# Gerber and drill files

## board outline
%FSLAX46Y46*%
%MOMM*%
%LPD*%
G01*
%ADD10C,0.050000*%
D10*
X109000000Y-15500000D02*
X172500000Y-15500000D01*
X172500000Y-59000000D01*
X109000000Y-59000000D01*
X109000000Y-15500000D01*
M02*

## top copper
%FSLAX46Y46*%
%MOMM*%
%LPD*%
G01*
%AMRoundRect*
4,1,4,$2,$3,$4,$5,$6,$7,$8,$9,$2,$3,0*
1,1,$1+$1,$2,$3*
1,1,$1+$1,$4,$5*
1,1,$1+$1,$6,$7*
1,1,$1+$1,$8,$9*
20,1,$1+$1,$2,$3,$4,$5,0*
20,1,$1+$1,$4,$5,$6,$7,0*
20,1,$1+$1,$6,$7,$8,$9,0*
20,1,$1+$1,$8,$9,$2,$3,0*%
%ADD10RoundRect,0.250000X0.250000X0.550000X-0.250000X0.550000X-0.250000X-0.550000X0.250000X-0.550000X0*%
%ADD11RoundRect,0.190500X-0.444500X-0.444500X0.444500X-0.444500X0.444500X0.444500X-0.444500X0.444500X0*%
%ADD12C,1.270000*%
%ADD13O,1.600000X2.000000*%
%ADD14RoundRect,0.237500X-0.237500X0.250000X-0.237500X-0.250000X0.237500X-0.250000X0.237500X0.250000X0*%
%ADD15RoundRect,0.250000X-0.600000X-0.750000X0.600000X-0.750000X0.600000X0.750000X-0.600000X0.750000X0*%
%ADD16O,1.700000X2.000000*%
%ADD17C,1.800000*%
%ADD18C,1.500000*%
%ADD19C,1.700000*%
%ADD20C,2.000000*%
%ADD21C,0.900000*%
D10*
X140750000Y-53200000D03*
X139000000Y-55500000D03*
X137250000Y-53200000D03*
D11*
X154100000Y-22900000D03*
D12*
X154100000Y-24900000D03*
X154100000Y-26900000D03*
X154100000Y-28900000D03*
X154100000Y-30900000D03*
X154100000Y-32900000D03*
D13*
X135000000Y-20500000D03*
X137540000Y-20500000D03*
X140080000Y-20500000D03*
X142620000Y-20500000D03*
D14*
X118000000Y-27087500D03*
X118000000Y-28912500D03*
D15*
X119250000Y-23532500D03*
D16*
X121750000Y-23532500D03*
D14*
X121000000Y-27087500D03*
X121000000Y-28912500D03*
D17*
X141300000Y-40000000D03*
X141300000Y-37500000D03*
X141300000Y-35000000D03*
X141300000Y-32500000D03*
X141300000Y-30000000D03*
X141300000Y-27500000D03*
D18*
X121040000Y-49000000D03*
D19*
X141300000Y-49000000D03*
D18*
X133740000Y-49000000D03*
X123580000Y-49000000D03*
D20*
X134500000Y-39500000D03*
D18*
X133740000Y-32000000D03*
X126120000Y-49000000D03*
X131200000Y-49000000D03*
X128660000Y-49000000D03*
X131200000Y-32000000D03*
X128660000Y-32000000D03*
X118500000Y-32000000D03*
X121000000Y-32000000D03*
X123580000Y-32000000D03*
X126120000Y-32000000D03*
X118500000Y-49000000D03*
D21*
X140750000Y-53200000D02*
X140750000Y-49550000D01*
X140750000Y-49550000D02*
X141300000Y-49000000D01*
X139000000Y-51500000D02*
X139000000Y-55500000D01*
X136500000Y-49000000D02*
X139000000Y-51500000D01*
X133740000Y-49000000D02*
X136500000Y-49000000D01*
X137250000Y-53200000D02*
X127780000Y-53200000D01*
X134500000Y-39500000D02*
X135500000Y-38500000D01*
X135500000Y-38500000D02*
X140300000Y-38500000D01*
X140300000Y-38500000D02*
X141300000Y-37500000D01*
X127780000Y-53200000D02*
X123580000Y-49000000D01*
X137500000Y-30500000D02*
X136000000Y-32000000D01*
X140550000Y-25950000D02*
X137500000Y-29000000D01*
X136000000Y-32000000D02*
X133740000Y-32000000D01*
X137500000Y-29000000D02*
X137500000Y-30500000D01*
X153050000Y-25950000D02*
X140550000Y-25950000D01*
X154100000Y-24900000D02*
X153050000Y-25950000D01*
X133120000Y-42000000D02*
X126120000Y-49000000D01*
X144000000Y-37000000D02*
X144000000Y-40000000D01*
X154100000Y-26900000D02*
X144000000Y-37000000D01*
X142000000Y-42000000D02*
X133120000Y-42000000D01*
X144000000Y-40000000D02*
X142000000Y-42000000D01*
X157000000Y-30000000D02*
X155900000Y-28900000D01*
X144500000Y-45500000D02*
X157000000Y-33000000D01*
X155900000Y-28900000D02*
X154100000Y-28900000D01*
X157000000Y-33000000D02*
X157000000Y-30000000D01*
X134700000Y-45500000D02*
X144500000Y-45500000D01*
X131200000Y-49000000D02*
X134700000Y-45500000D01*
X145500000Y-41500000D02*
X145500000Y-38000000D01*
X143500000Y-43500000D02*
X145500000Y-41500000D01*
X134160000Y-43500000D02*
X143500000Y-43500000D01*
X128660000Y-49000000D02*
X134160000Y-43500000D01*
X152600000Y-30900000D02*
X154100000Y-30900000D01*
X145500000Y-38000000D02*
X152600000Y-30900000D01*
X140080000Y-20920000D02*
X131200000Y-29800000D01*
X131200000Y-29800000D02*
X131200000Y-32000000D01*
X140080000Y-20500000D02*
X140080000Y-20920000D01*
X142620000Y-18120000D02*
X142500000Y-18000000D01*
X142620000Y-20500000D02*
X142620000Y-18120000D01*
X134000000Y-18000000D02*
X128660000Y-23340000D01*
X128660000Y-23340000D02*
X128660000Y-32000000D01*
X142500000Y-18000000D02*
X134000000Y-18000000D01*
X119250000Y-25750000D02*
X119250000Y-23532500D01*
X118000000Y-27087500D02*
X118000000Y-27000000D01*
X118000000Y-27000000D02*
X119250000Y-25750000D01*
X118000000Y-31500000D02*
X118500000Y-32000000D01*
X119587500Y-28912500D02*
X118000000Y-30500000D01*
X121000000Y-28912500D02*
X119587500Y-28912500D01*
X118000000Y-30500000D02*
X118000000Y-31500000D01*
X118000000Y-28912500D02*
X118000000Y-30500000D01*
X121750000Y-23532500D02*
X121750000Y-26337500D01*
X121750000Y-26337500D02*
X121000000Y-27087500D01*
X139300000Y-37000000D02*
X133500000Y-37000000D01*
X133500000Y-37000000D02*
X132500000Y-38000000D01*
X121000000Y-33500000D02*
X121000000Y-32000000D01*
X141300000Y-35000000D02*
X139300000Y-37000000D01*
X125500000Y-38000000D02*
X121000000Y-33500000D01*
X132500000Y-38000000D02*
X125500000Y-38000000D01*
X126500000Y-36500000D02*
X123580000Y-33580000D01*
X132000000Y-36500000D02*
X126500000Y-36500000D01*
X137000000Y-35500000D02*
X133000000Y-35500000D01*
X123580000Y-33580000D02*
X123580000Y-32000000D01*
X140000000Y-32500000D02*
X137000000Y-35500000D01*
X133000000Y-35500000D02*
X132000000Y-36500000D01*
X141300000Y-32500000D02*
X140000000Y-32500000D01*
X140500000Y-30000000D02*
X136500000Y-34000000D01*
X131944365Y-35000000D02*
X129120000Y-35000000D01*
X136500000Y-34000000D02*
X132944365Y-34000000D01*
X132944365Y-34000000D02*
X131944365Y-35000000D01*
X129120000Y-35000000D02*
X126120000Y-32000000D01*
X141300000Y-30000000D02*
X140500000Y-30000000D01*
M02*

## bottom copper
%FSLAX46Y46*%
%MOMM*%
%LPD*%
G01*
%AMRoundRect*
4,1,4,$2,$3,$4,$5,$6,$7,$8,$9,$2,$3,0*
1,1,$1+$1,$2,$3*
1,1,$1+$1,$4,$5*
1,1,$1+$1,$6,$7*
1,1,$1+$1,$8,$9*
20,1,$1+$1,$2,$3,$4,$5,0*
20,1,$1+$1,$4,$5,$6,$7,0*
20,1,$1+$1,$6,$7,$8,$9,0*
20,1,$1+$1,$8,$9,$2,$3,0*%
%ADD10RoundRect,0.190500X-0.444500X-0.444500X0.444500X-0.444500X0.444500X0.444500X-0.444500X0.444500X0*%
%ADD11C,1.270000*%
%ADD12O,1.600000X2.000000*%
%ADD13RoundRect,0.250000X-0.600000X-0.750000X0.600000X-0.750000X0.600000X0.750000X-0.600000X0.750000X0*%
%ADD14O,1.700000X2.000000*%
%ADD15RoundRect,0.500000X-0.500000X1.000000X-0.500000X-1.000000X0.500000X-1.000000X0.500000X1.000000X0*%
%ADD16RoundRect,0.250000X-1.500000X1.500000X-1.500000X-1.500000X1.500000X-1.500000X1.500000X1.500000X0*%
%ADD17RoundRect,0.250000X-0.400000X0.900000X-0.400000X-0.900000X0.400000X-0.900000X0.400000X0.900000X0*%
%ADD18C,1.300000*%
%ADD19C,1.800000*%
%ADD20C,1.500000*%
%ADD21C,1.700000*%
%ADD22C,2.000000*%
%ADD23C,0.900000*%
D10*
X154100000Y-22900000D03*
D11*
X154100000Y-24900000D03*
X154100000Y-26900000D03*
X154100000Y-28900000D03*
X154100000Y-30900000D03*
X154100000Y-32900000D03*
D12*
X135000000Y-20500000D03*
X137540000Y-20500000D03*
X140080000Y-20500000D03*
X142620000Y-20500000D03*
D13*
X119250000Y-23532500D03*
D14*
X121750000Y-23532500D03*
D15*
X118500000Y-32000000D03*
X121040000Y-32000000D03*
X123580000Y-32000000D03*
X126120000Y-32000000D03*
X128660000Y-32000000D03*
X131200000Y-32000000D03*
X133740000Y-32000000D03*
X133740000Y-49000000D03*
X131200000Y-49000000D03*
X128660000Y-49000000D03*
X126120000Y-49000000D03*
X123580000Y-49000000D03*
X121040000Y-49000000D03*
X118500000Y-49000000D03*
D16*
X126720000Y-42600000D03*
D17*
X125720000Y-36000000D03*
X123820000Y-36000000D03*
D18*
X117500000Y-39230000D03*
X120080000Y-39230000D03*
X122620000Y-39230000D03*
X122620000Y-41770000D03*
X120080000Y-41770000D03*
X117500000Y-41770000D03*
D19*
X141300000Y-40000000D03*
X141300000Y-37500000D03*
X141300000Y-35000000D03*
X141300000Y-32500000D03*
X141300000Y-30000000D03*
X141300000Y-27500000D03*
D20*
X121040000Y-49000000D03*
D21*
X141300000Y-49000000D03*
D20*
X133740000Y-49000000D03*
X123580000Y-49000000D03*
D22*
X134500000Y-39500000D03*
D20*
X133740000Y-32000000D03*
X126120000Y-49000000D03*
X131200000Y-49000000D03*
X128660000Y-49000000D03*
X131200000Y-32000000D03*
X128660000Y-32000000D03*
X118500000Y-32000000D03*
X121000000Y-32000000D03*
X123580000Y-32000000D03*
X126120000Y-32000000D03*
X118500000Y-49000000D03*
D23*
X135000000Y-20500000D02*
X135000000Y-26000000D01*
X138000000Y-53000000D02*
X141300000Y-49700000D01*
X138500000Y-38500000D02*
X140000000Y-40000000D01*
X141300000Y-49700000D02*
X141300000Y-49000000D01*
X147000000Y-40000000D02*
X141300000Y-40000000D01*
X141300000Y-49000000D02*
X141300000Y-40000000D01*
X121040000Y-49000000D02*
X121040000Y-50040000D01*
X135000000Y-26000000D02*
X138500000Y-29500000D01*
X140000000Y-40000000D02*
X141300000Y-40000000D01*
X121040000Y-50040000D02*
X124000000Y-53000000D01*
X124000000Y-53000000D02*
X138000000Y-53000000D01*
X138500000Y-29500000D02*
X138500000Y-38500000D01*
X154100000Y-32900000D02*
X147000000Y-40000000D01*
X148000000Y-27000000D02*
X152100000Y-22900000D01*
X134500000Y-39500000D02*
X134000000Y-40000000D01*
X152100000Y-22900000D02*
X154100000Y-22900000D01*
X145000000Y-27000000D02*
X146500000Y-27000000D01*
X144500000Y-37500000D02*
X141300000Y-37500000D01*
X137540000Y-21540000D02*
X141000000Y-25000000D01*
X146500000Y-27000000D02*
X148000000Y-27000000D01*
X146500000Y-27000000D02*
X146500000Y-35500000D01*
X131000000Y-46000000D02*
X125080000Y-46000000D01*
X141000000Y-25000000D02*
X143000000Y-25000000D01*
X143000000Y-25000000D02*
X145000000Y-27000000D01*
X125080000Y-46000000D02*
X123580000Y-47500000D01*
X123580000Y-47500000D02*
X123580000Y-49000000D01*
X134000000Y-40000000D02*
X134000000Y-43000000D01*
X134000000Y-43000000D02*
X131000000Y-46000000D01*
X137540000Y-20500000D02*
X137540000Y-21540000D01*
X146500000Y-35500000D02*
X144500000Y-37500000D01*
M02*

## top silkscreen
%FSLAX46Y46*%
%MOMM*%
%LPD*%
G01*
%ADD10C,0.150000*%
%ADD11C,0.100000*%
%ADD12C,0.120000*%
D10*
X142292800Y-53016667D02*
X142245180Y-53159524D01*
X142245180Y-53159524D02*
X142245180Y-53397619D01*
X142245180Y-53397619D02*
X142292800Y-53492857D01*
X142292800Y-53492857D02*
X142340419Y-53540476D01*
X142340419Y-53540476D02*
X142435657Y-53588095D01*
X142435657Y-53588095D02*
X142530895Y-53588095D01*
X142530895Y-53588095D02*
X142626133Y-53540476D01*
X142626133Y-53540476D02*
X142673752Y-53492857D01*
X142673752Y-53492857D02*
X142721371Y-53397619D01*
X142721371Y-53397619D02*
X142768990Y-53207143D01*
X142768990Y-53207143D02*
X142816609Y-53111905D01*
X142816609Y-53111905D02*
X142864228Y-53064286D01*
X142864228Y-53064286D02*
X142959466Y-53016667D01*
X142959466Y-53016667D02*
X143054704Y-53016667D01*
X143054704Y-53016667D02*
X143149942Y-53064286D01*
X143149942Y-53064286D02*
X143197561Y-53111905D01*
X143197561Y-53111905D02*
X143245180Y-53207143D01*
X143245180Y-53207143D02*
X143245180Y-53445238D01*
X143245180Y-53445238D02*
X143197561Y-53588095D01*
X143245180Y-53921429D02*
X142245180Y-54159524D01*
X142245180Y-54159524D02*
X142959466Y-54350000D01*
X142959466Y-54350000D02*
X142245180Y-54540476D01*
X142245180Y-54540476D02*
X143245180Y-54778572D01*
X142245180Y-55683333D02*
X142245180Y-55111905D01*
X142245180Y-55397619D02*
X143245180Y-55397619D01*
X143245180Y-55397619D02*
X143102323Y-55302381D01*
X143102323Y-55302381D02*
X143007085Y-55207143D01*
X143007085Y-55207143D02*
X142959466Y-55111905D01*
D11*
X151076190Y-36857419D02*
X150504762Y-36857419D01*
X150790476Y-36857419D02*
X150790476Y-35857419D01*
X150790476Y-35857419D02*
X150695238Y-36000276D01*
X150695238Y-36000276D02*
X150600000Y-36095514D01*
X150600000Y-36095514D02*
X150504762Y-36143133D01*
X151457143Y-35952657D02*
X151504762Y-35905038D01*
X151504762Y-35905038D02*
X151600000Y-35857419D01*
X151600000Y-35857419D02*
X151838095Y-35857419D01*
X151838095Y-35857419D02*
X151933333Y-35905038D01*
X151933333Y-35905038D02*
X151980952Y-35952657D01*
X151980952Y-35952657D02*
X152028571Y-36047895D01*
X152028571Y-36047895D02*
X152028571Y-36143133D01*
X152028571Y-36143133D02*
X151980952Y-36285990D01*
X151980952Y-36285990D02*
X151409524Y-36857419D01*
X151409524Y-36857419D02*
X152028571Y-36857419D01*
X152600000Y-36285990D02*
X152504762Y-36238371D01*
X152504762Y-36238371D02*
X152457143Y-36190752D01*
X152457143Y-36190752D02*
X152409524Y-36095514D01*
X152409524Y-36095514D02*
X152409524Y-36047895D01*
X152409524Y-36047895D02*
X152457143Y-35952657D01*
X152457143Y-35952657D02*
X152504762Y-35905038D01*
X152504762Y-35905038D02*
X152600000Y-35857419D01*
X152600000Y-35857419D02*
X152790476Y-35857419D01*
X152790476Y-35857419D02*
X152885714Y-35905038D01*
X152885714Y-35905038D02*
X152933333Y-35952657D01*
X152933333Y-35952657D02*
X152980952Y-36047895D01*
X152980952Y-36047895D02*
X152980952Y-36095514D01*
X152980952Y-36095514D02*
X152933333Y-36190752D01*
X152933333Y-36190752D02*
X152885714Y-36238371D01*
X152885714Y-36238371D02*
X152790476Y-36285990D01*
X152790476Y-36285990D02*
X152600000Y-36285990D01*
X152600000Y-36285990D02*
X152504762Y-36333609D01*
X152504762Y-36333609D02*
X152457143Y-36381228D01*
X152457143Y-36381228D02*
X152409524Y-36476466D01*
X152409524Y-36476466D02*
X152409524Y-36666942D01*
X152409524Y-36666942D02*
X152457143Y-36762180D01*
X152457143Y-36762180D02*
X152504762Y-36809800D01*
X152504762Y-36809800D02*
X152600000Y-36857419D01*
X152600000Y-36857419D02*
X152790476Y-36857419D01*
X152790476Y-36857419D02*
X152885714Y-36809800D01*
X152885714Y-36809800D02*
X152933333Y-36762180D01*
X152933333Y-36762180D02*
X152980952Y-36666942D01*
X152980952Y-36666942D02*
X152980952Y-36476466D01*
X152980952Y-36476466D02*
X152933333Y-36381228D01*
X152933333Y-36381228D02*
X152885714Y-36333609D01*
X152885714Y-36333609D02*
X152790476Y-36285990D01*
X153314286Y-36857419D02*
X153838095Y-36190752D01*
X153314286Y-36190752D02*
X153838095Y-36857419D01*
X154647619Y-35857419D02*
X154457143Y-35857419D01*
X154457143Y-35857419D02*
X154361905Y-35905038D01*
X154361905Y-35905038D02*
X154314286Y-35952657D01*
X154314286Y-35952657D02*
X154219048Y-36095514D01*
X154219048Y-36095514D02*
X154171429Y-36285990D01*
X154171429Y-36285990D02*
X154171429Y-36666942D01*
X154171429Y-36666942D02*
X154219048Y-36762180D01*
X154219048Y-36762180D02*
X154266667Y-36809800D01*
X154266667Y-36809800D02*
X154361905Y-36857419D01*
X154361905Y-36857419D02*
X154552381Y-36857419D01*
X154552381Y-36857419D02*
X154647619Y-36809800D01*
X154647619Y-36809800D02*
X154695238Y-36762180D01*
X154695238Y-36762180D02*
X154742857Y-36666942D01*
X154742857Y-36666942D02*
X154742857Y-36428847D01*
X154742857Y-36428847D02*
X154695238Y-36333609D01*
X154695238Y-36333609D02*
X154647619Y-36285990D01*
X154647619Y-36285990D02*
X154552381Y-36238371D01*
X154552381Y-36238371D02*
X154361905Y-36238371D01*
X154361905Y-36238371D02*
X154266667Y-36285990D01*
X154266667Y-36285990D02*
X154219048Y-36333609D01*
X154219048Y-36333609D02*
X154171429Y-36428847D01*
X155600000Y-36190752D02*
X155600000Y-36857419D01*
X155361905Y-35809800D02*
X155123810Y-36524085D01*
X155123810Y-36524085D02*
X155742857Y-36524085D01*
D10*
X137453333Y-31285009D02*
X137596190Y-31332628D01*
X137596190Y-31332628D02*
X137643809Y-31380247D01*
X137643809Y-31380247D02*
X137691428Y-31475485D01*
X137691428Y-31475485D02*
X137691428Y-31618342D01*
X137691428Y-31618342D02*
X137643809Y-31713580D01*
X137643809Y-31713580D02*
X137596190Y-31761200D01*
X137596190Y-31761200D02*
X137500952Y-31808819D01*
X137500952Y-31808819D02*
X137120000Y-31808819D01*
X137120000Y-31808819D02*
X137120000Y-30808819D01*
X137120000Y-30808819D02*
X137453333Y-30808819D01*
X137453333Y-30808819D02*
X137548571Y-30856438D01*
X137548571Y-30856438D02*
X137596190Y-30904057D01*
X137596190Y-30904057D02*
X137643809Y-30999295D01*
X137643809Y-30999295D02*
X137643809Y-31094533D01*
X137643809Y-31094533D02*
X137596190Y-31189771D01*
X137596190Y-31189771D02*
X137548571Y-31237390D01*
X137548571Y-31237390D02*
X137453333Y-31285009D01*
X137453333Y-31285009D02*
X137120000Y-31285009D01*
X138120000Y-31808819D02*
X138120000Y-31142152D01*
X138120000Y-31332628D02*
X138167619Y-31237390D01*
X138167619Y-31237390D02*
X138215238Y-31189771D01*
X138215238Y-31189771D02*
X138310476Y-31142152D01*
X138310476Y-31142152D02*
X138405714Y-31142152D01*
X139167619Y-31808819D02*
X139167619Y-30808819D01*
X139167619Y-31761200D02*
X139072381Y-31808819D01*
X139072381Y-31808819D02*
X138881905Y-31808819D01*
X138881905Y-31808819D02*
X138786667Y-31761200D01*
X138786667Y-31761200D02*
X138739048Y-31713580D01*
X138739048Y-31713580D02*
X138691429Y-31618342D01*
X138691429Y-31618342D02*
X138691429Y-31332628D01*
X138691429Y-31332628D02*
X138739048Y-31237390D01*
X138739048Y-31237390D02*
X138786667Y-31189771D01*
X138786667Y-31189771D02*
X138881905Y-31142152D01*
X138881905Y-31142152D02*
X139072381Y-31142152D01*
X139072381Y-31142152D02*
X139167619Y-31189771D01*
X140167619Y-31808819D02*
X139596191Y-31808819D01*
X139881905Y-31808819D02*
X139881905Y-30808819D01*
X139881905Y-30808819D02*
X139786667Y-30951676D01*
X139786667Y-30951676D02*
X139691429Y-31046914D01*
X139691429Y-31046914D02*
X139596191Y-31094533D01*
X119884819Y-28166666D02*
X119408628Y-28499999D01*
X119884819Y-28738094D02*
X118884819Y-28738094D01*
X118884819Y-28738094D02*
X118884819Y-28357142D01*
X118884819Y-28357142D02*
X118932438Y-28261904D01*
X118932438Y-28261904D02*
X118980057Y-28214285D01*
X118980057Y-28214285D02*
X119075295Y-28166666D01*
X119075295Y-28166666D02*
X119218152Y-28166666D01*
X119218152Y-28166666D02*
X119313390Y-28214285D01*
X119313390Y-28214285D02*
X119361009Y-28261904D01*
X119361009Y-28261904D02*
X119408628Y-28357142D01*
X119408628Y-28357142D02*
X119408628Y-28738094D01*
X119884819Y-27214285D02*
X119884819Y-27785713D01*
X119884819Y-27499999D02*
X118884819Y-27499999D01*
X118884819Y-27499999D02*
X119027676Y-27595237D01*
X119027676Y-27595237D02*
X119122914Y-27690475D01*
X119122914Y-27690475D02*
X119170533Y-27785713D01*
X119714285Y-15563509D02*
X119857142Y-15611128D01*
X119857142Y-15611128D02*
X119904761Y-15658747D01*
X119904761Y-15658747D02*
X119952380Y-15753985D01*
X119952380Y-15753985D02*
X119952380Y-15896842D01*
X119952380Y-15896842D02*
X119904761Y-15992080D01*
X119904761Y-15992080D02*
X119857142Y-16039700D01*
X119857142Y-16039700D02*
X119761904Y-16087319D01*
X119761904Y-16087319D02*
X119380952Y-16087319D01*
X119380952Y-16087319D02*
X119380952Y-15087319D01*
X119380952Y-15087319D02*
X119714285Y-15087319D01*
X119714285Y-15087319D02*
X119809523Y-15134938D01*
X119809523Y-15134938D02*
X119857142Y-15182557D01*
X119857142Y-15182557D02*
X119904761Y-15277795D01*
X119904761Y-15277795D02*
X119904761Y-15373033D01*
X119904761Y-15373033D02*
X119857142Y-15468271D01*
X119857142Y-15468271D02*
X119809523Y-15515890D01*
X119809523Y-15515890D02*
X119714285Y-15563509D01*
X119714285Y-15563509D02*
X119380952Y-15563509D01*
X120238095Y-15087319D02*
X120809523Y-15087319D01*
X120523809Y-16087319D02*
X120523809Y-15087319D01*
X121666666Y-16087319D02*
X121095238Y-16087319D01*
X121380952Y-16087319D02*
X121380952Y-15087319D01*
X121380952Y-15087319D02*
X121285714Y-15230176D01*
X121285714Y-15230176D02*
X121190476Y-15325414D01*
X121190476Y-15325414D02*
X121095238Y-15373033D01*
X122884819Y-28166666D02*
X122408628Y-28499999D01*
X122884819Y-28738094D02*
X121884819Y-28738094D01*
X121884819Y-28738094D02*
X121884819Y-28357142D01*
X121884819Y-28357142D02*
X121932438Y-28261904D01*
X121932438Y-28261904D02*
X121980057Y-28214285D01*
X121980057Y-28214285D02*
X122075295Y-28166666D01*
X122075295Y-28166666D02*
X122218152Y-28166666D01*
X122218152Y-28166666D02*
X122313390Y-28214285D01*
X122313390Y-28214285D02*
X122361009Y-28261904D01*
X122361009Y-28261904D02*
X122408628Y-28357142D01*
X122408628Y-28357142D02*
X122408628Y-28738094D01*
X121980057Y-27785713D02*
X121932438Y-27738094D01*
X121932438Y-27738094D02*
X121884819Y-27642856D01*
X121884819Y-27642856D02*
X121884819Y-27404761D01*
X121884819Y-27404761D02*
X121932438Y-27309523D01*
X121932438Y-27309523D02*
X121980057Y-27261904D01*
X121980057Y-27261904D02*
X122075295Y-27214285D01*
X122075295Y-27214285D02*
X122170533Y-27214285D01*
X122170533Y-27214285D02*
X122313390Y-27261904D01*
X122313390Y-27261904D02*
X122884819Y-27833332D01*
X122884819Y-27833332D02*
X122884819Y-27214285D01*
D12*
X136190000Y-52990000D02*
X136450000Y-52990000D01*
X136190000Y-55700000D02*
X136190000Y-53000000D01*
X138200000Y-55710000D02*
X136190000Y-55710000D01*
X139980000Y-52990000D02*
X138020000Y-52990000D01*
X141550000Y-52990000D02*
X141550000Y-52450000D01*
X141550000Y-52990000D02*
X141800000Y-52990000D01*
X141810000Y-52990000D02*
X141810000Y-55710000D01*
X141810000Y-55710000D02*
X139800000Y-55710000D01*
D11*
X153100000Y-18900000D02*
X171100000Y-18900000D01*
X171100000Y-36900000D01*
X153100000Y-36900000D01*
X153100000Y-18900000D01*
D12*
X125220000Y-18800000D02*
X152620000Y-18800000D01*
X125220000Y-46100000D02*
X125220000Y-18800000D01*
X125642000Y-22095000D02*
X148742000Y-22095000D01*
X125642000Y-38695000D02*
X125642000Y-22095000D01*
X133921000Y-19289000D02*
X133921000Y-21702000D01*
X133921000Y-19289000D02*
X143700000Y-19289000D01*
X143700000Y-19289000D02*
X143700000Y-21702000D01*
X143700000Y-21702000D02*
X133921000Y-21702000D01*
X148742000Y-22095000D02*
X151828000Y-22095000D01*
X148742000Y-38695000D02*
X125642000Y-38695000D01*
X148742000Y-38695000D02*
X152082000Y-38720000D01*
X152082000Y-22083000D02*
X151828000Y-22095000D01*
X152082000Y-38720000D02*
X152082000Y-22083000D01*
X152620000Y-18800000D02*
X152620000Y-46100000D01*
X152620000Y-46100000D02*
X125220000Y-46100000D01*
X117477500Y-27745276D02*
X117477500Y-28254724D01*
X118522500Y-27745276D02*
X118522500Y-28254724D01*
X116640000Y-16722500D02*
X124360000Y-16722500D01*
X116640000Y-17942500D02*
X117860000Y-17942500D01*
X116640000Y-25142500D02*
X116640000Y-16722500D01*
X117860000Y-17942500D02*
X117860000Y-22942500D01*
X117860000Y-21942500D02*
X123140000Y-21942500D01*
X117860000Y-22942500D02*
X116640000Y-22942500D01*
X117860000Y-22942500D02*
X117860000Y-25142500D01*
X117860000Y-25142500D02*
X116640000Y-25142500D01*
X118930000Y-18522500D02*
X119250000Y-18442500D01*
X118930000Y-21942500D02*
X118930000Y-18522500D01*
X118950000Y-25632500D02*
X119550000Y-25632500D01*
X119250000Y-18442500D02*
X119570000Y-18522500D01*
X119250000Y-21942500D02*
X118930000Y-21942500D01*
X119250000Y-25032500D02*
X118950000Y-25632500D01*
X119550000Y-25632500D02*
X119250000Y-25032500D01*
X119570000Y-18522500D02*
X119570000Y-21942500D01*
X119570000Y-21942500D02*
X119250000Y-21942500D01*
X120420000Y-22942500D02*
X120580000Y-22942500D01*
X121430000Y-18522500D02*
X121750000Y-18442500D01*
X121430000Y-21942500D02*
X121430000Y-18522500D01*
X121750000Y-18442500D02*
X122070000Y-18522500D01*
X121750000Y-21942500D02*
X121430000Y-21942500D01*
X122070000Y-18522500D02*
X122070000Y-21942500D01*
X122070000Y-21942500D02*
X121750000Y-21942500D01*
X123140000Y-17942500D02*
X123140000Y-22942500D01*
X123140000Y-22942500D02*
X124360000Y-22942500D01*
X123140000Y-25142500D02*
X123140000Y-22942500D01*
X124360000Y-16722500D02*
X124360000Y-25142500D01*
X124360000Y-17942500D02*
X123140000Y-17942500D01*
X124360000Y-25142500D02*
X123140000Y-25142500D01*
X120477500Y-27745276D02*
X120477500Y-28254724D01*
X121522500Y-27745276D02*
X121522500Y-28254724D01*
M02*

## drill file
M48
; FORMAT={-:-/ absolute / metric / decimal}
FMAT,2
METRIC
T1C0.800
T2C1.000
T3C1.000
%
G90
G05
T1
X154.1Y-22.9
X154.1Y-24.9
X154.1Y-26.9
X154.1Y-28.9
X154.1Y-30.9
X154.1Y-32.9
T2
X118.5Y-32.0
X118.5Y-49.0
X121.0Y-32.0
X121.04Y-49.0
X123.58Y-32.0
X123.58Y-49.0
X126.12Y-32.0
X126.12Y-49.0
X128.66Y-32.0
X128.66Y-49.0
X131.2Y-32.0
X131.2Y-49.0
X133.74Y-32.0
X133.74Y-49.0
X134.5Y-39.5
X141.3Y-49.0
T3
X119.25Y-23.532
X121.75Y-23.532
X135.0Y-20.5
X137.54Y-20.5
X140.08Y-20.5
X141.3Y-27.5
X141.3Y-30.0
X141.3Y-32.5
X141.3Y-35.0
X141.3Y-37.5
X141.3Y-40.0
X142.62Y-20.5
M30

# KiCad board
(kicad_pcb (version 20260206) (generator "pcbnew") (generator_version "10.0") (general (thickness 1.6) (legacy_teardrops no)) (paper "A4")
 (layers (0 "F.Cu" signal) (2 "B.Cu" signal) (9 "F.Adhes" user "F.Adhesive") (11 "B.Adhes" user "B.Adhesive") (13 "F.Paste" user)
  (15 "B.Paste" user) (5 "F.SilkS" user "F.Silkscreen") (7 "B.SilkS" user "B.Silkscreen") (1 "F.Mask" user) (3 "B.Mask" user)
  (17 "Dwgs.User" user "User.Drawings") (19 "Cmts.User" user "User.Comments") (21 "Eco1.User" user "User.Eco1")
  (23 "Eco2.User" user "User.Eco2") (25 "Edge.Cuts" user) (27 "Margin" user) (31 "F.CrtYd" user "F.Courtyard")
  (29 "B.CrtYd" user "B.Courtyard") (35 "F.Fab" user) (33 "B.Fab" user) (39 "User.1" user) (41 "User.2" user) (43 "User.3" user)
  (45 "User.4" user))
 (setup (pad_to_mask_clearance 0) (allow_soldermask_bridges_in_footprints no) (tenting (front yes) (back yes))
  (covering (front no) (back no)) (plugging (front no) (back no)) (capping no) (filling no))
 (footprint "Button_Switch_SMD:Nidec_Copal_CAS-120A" (layer "F.Cu") (at 139 54.35 -90)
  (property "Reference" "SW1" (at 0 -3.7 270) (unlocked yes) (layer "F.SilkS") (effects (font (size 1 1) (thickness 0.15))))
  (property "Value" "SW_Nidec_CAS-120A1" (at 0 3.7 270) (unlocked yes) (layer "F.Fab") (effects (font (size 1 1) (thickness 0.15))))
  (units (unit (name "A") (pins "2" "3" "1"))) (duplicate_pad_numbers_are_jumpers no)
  (fp_line (start -1.36 2.81) (end -1.36 2.55) (stroke (width 0.12) (type solid)) (layer "F.SilkS"))
  (fp_line (start 1.35 2.81) (end -1.35 2.81) (stroke (width 0.12) (type solid)) (layer "F.SilkS"))
  (fp_line (start 1.36 0.8) (end 1.36 2.81) (stroke (width 0.12) (type solid)) (layer "F.SilkS"))
  (fp_line (start -1.36 -0.98) (end -1.36 0.98) (stroke (width 0.12) (type solid)) (layer "F.SilkS"))
  (fp_line (start -1.36 -2.55) (end -1.9 -2.55) (stroke (width 0.12) (type default)) (layer "F.SilkS"))
  (fp_line (start -1.36 -2.55) (end -1.36 -2.8) (stroke (width 0.12) (type solid)) (layer "F.SilkS"))
  (fp_line (start -1.36 -2.81) (end 1.36 -2.81) (stroke (width 0.12) (type solid)) (layer "F.SilkS"))
  (fp_line (start 1.36 -2.81) (end 1.36 -0.8) (stroke (width 0.12) (type solid)) (layer "F.SilkS"))
  (pad "1" smd roundrect (at -1.15 -1.75 180) (size 1 1.6) (layers "F.Cu" "F.Mask" "F.Paste") (roundrect_rratio 0.25) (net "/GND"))
  (pad "2" smd roundrect (at 1.15 0 180) (size 1 1.6) (layers "F.Cu" "F.Mask" "F.Paste") (roundrect_rratio 0.25) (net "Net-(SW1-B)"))
  (pad "3" smd roundrect (at -1.15 1.75 180) (size 1 1.6) (layers "F.Cu" "F.Mask" "F.Paste") (roundrect_rratio 0.25) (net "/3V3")))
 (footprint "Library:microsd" (layer "F.Cu") (at 153.1 36.9)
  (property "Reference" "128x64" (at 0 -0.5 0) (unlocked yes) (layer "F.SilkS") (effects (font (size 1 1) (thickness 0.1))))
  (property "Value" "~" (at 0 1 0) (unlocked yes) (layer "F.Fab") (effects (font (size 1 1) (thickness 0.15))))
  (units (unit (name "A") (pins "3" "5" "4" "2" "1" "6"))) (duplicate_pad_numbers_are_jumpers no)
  (fp_rect (start 0 -18) (end 18 0) (stroke (width 0.1) (type default)) (fill no) (layer "F.SilkS"))
  (pad "1" thru_hole roundrect (at 1 -14) (size 1.27 1.27) (drill 0.8) (layers "*.Cu" "*.Mask") (remove_unused_layers no)
   (roundrect_rratio 0.15) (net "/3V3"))
  (pad "2" thru_hole circle (at 1 -12) (size 1.27 1.27) (drill 0.8) (layers "*.Cu" "*.Mask") (remove_unused_layers no) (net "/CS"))
  (pad "3" thru_hole circle (at 1 -10) (size 1.27 1.27) (drill 0.8) (layers "*.Cu" "*.Mask") (remove_unused_layers no) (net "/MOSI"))
  (pad "4" thru_hole circle (at 1 -8) (size 1.27 1.27) (drill 0.8) (layers "*.Cu" "*.Mask") (remove_unused_layers no) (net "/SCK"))
  (pad "5" thru_hole circle (at 1 -6) (size 1.27 1.27) (drill 0.8) (layers "*.Cu" "*.Mask") (remove_unused_layers no) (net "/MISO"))
  (pad "6" thru_hole circle (at 1 -4) (size 1.27 1.27) (drill 0.8) (layers "*.Cu" "*.Mask") (remove_unused_layers no) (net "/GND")))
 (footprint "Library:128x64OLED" (layer "F.Cu") (at 138.62 31.1)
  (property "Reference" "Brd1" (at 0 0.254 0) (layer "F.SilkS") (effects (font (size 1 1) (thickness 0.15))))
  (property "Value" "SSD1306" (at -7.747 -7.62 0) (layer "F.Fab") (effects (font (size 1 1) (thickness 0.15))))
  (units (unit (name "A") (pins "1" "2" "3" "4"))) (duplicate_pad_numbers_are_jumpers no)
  (fp_line (start -13.4 -12.3) (end 14 -12.3) (stroke (width 0.12) (type solid)) (layer "F.SilkS"))
  (fp_line (start -13.4 15) (end -13.4 -12.3) (stroke (width 0.12) (type solid)) (layer "F.SilkS"))
  (fp_line (start -12.978 -9.005) (end 10.122 -9.005) (stroke (width 0.12) (type solid)) (layer "F.SilkS"))
  (fp_line (start -12.978 7.595) (end -12.978 -9.005) (stroke (width 0.12) (type solid)) (layer "F.SilkS"))
  (fp_line (start -4.699 -11.811) (end -4.699 -9.398) (stroke (width 0.12) (type solid)) (layer "F.SilkS"))
  (fp_line (start -4.699 -11.811) (end 5.08 -11.811) (stroke (width 0.12) (type solid)) (layer "F.SilkS"))
  (fp_line (start 5.08 -11.811) (end 5.08 -9.398) (stroke (width 0.12) (type solid)) (layer "F.SilkS"))
  (fp_line (start 5.08 -9.398) (end -4.699 -9.398) (stroke (width 0.12) (type solid)) (layer "F.SilkS"))
  (fp_line (start 10.122 -9.005) (end 13.208 -9.005) (stroke (width 0.12) (type solid)) (layer "F.SilkS"))
  (fp_line (start 10.122 7.595) (end -12.978 7.595) (stroke (width 0.12) (type solid)) (layer "F.SilkS"))
  (fp_line (start 10.122 7.595) (end 13.462 7.62) (stroke (width 0.12) (type solid)) (layer "F.SilkS"))
  (fp_line (start 13.462 -9.017) (end 13.208 -9.005) (stroke (width 0.12) (type solid)) (layer "F.SilkS"))
  (fp_line (start 13.462 7.62) (end 13.462 -9.017) (stroke (width 0.12) (type solid)) (layer "F.SilkS"))
  (fp_line (start 14 -12.3) (end 14 15) (stroke (width 0.12) (type solid)) (layer "F.SilkS"))
  (fp_line (start 14 15) (end -13.4 15) (stroke (width 0.12) (type solid)) (layer "F.SilkS"))
  (pad "1" thru_hole oval (at -3.62 -10.6 90) (size 2 1.6) (drill 1) (layers "*.Cu" "*.Mask") (remove_unused_layers no) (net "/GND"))
  (pad "2" thru_hole oval (at -1.08 -10.6 90) (size 2 1.6) (drill 1) (layers "*.Cu" "*.Mask") (remove_unused_layers no) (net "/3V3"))
  (pad "3" thru_hole oval (at 1.46 -10.6 90) (size 2 1.6) (drill 1) (layers "*.Cu" "*.Mask") (remove_unused_layers no) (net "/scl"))
  (pad "4" thru_hole oval (at 4 -10.6 90) (size 2 1.6) (drill 1) (layers "*.Cu" "*.Mask") (remove_unused_layers no) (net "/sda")))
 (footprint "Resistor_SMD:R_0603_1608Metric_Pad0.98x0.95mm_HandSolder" (layer "F.Cu") (at 118 28 -90)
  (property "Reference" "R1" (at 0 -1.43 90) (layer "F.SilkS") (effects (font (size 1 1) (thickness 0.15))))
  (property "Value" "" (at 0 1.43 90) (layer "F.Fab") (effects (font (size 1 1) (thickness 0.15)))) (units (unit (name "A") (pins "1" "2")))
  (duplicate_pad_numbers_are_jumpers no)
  (fp_line (start -0.254724 0.5225) (end 0.254724 0.5225) (stroke (width 0.12) (type solid)) (layer "F.SilkS"))
  (fp_line (start -0.254724 -0.5225) (end 0.254724 -0.5225) (stroke (width 0.12) (type solid)) (layer "F.SilkS"))
  (pad "1" smd roundrect (at -0.9125 0 270) (size 0.975 0.95) (layers "F.Cu" "F.Mask" "F.Paste") (roundrect_rratio 0.25) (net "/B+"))
  (pad "2" smd roundrect (at 0.9125 0 270) (size 0.975 0.95) (layers "F.Cu" "F.Mask" "F.Paste") (roundrect_rratio 0.25) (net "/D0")))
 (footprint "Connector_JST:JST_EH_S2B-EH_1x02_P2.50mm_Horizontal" (layer "F.Cu") (at 119.25 23.5325)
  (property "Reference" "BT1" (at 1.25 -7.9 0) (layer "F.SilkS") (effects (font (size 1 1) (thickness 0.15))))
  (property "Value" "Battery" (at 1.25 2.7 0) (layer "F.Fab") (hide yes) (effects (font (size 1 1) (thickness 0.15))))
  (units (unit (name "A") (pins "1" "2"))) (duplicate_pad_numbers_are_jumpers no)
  (fp_line (start -2.61 -6.81) (end 5.11 -6.81) (stroke (width 0.12) (type solid)) (layer "F.SilkS"))
  (fp_line (start -2.61 -5.59) (end -1.39 -5.59) (stroke (width 0.12) (type solid)) (layer "F.SilkS"))
  (fp_line (start -2.61 1.61) (end -2.61 -6.81) (stroke (width 0.12) (type solid)) (layer "F.SilkS"))
  (fp_line (start -1.39 -5.59) (end -1.39 -0.59) (stroke (width 0.12) (type solid)) (layer "F.SilkS"))
  (fp_line (start -1.39 -1.59) (end 3.89 -1.59) (stroke (width 0.12) (type solid)) (layer "F.SilkS"))
  (fp_line (start -1.39 -0.59) (end -2.61 -0.59) (stroke (width 0.12) (type solid)) (layer "F.SilkS"))
  (fp_line (start -1.39 -0.59) (end -1.39 1.61) (stroke (width 0.12) (type solid)) (layer "F.SilkS"))
  (fp_line (start -1.39 1.61) (end -2.61 1.61) (stroke (width 0.12) (type solid)) (layer "F.SilkS"))
  (fp_line (start -0.32 -5.01) (end 0 -5.09) (stroke (width 0.12) (type solid)) (layer "F.SilkS"))
  (fp_line (start -0.32 -1.59) (end -0.32 -5.01) (stroke (width 0.12) (type solid)) (layer "F.SilkS"))
  (fp_line (start -0.3 2.1) (end 0.3 2.1) (stroke (width 0.12) (type solid)) (layer "F.SilkS"))
  (fp_line (start 0 -5.09) (end 0.32 -5.01) (stroke (width 0.12) (type solid)) (layer "F.SilkS"))
  (fp_line (start 0 -1.59) (end -0.32 -1.59) (stroke (width 0.12) (type solid)) (layer "F.SilkS"))
  (fp_line (start 0 1.5) (end -0.3 2.1) (stroke (width 0.12) (type solid)) (layer "F.SilkS"))
  (fp_line (start 0.3 2.1) (end 0 1.5) (stroke (width 0.12) (type solid)) (layer "F.SilkS"))
  (fp_line (start 0.32 -5.01) (end 0.32 -1.59) (stroke (width 0.12) (type solid)) (layer "F.SilkS"))
  (fp_line (start 0.32 -1.59) (end 0 -1.59) (stroke (width 0.12) (type solid)) (layer "F.SilkS"))
  (fp_line (start 1.17 -0.59) (end 1.33 -0.59) (stroke (width 0.12) (type solid)) (layer "F.SilkS"))
  (fp_line (start 2.18 -5.01) (end 2.5 -5.09) (stroke (width 0.12) (type solid)) (layer "F.SilkS"))
  (fp_line (start 2.18 -1.59) (end 2.18 -5.01) (stroke (width 0.12) (type solid)) (layer "F.SilkS"))
  (fp_line (start 2.5 -5.09) (end 2.82 -5.01) (stroke (width 0.12) (type solid)) (layer "F.SilkS"))
  (fp_line (start 2.5 -1.59) (end 2.18 -1.59) (stroke (width 0.12) (type solid)) (layer "F.SilkS"))
  (fp_line (start 2.82 -5.01) (end 2.82 -1.59) (stroke (width 0.12) (type solid)) (layer "F.SilkS"))
  (fp_line (start 2.82 -1.59) (end 2.5 -1.59) (stroke (width 0.12) (type solid)) (layer "F.SilkS"))
  (fp_line (start 3.89 -5.59) (end 3.89 -0.59) (stroke (width 0.12) (type solid)) (layer "F.SilkS"))
  (fp_line (start 3.89 -0.59) (end 5.11 -0.59) (stroke (width 0.12) (type solid)) (layer "F.SilkS"))
  (fp_line (start 3.89 1.61) (end 3.89 -0.59) (stroke (width 0.12) (type solid)) (layer "F.SilkS"))
  (fp_line (start 5.11 -6.81) (end 5.11 1.61) (stroke (width 0.12) (type solid)) (layer "F.SilkS"))
  (fp_line (start 5.11 -5.59) (end 3.89 -5.59) (stroke (width 0.12) (type solid)) (layer "F.SilkS"))
  (fp_line (start 5.11 1.61) (end 3.89 1.61) (stroke (width 0.12) (type solid)) (layer "F.SilkS"))
  (pad "1" thru_hole roundrect (at 0 0) (size 1.7 2) (drill 1) (layers "*.Cu" "*.Mask") (remove_unused_layers no)
   (roundrect_rratio 0.147059) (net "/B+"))
  (pad "2" thru_hole oval (at 2.5 0) (size 1.7 2) (drill 1) (layers "*.Cu" "*.Mask") (remove_unused_layers no) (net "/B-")))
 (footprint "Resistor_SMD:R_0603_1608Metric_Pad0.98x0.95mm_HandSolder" (layer "F.Cu") (at 121 28 -90)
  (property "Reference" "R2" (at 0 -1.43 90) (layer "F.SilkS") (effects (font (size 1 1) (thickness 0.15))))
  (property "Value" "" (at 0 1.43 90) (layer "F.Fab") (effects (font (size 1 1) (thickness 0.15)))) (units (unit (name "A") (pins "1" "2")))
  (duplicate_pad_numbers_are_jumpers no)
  (fp_line (start -0.254724 0.5225) (end 0.254724 0.5225) (stroke (width 0.12) (type solid)) (layer "F.SilkS"))
  (fp_line (start -0.254724 -0.5225) (end 0.254724 -0.5225) (stroke (width 0.12) (type solid)) (layer "F.SilkS"))
  (pad "1" smd roundrect (at -0.9125 0 270) (size 0.975 0.95) (layers "F.Cu" "F.Mask" "F.Paste") (roundrect_rratio 0.25) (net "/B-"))
  (pad "2" smd roundrect (at 0.9125 0 270) (size 0.975 0.95) (layers "F.Cu" "F.Mask" "F.Paste") (roundrect_rratio 0.25) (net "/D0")))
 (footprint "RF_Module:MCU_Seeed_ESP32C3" (layer "B.Cu") (at 126.12 40.5 -90)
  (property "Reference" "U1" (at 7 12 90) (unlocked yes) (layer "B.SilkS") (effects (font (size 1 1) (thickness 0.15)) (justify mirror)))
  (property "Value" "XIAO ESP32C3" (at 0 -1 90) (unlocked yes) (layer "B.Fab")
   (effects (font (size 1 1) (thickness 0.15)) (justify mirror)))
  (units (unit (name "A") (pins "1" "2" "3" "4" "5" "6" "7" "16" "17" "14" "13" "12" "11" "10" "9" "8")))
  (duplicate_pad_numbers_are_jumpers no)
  (pad "" smd roundrect (at 1.1 -1.6 270) (size 1.5 1.5) (layers "B.Paste") (roundrect_rratio 0.1666666667))
  (pad "" smd roundrect (at 1.1 0.4 270) (size 1.5 1.5) (layers "B.Paste") (roundrect_rratio 0.1666666667))
  (pad "" smd roundrect (at 3.1 -1.6 270) (size 1.5 1.5) (layers "B.Paste") (roundrect_rratio 0.1666666667))
  (pad "" smd roundrect (at 3.1 0.4 270) (size 1.5 1.5) (layers "B.Paste") (roundrect_rratio 0.1666666667))
  (pad "1" smd roundrect (at -8.5 7.62 270) (size 3 2) (layers "B.Cu" "B.Mask" "B.Paste") (roundrect_rratio 0.25) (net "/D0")
   (thermal_bridge_angle 45))
  (pad "2" smd roundrect (at -8.5 5.08 270) (size 3 2) (layers "B.Cu" "B.Mask" "B.Paste") (roundrect_rratio 0.25) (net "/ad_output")
   (thermal_bridge_angle 45))
  (pad "3" smd roundrect (at -8.5 2.54 270) (size 3 2) (layers "B.Cu" "B.Mask" "B.Paste") (roundrect_rratio 0.25) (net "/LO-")
   (thermal_bridge_angle 45))
  (pad "4" smd roundrect (at -8.5 0 270) (size 3 2) (layers "B.Cu" "B.Mask" "B.Paste") (roundrect_rratio 0.25) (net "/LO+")
   (thermal_bridge_angle 45))
  (pad "5" smd roundrect (at -8.5 -2.54 270) (size 3 2) (layers "B.Cu" "B.Mask" "B.Paste") (roundrect_rratio 0.25) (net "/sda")
   (thermal_bridge_angle 45))
  (pad "6" smd roundrect (at -8.5 -5.08 270) (size 3 2) (layers "B.Cu" "B.Mask" "B.Paste") (roundrect_rratio 0.25) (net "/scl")
   (thermal_bridge_angle 45))
  (pad "7" smd roundrect (at -8.5 -7.62 270) (size 3 2) (layers "B.Cu" "B.Mask" "B.Paste") (roundrect_rratio 0.25) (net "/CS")
   (thermal_bridge_angle 45))
  (pad "8" smd roundrect (at 8.5 -7.62 270) (size 3 2) (layers "B.Cu" "B.Mask" "B.Paste") (roundrect_rratio 0.25) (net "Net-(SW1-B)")
   (thermal_bridge_angle 45))
  (pad "9" smd roundrect (at 8.5 -5.08 270) (size 3 2) (layers "B.Cu" "B.Mask" "B.Paste") (roundrect_rratio 0.25) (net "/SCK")
   (thermal_bridge_angle 45))
  (pad "10" smd roundrect (at 8.5 -2.54 270) (size 3 2) (layers "B.Cu" "B.Mask" "B.Paste") (roundrect_rratio 0.25) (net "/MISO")
   (thermal_bridge_angle 45))
  (pad "11" smd roundrect (at 8.5 0 270) (size 3 2) (layers "B.Cu" "B.Mask" "B.Paste") (roundrect_rratio 0.25) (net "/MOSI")
   (thermal_bridge_angle 45))
  (pad "12" smd roundrect (at 8.5 2.54 270) (size 3 2) (layers "B.Cu" "B.Mask" "B.Paste") (roundrect_rratio 0.25) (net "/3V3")
   (thermal_bridge_angle 45))
  (pad "13" smd roundrect (at 8.5 5.08 270) (size 3 2) (layers "B.Cu" "B.Mask" "B.Paste") (roundrect_rratio 0.25) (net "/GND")
   (thermal_bridge_angle 45))
  (pad "14" smd roundrect (at 8.5 7.62 270) (size 3 2) (layers "B.Cu" "B.Mask" "B.Paste") (roundrect_rratio 0.25)
   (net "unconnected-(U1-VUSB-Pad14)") (thermal_bridge_angle 45))
  (pad "15" smd roundrect (at 2.1 -0.6 270) (size 3.5 3.5) (layers "B.Cu" "B.Mask") (roundrect_rratio 0.07142857143))
  (pad "16" smd roundrect (at -4.5 0.4 270) (size 2.3 1.3) (layers "B.Cu" "B.Mask" "B.Paste") (roundrect_rratio 0.1923076923) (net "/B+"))
  (pad "17" smd roundrect (at -4.5 2.3 270) (size 2.3 1.3) (layers "B.Cu" "B.Mask" "B.Paste") (roundrect_rratio 0.1923076923) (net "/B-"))
  (pad "18" smd circle (at -1.27 8.62 270) (size 1.3 1.3) (layers "B.Cu" "B.Mask" "B.Paste"))
  (pad "19" smd circle (at -1.27 6.04 270) (size 1.3 1.3) (layers "B.Cu" "B.Mask" "B.Paste"))
  (pad "20" smd circle (at -1.27 3.5 270) (size 1.3 1.3) (layers "B.Cu" "B.Mask" "B.Paste"))
  (pad "21" smd circle (at 1.27 3.5 270) (size 1.3 1.3) (layers "B.Cu" "B.Mask" "B.Paste"))
  (pad "22" smd circle (at 1.27 6.04 270) (size 1.3 1.3) (layers "B.Cu" "B.Mask" "B.Paste"))
  (pad "23" smd circle (at 1.27 8.62 270) (size 1.3 1.3) (layers "B.Cu" "B.Mask" "B.Paste")))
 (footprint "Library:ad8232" (layer "B.Cu") (at 140.1 19)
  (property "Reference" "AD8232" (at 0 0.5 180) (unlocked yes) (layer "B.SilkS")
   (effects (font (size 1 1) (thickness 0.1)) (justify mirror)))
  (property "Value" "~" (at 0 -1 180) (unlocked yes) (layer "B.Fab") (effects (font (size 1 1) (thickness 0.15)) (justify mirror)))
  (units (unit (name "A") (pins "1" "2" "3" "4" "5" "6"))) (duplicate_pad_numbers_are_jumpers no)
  (pad "1" thru_hole circle (at 1.2 21) (size 1.8 1.8) (drill 1) (layers "*.Cu" "*.Mask") (remove_unused_layers no) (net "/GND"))
  (pad "2" thru_hole circle (at 1.2 18.5) (size 1.8 1.8) (drill 1) (layers "*.Cu" "*.Mask") (remove_unused_layers no) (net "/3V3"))
  (pad "3" thru_hole circle (at 1.2 16) (size 1.8 1.8) (drill 1) (layers "*.Cu" "*.Mask") (remove_unused_layers no) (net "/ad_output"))
  (pad "4" thru_hole circle (at 1.2 13.5) (size 1.8 1.8) (drill 1) (layers "*.Cu" "*.Mask") (remove_unused_layers no) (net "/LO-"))
  (pad "5" thru_hole circle (at 1.2 11) (size 1.8 1.8) (drill 1) (layers "*.Cu" "*.Mask") (remove_unused_layers no) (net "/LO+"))
  (pad "6" thru_hole circle (at 1.2 8.5) (size 1.8 1.8) (drill 1) (layers "*.Cu" "*.Mask") (remove_unused_layers no)
   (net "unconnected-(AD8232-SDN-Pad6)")))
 (gr_rect (start 109 15.5) (end 172.5 59) (stroke (width 0.05) (type default)) (fill no) (layer "Edge.Cuts"))
 (segment (start 140.75 53.2) (end 140.75 49.55) (width 0.9) (layer "F.Cu") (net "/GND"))
 (segment (start 140.75 49.55) (end 141.3 49) (width 0.9) (layer "F.Cu") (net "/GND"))
 (via (at 121.04 49) (size 1.5) (drill 1) (layers "F.Cu" "B.Cu") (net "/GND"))
 (via (at 141.3 49) (size 1.7) (drill 1) (layers "F.Cu" "B.Cu") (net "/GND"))
 (segment (start 135 20.5) (end 135 26) (width 0.9) (layer "B.Cu") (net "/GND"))
 (segment (start 138 53) (end 141.3 49.7) (width 0.9) (layer "B.Cu") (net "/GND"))
 (segment (start 138.5 38.5) (end 140 40) (width 0.9) (layer "B.Cu") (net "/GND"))
 (segment (start 141.3 49.7) (end 141.3 49) (width 0.9) (layer "B.Cu") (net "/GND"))
 (segment (start 147 40) (end 141.3 40) (width 0.9) (layer "B.Cu") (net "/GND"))
 (segment (start 141.3 49) (end 141.3 40) (width 0.9) (layer "B.Cu") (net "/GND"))
 (segment (start 121.04 49) (end 121.04 50.04) (width 0.9) (layer "B.Cu") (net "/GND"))
 (segment (start 135 26) (end 138.5 29.5) (width 0.9) (layer "B.Cu") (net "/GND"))
 (segment (start 140 40) (end 141.3 40) (width 0.9) (layer "B.Cu") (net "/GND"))
 (segment (start 121.04 50.04) (end 124 53) (width 0.9) (layer "B.Cu") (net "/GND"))
 (segment (start 124 53) (end 138 53) (width 0.9) (layer "B.Cu") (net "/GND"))
 (segment (start 138.5 29.5) (end 138.5 38.5) (width 0.9) (layer "B.Cu") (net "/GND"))
 (segment (start 154.1 32.9) (end 147 40) (width 0.9) (layer "B.Cu") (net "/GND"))
 (segment (start 139 51.5) (end 139 55.5) (width 0.9) (layer "F.Cu") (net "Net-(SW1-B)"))
 (segment (start 136.5 49) (end 139 51.5) (width 0.9) (layer "F.Cu") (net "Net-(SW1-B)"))
 (segment (start 133.74 49) (end 136.5 49) (width 0.9) (layer "F.Cu") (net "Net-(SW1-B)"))
 (via (at 133.74 49) (size 1.5) (drill 1) (layers "F.Cu" "B.Cu") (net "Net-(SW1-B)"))
 (segment (start 137.25 53.2) (end 127.78 53.2) (width 0.9) (layer "F.Cu") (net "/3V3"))
 (segment (start 134.5 39.5) (end 135.5 38.5) (width 0.9) (layer "F.Cu") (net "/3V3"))
 (segment (start 135.5 38.5) (end 140.3 38.5) (width 0.9) (layer "F.Cu") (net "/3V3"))
 (segment (start 140.3 38.5) (end 141.3 37.5) (width 0.9) (layer "F.Cu") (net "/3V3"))
 (segment (start 127.78 53.2) (end 123.58 49) (width 0.9) (layer "F.Cu") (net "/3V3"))
 (via (at 123.58 49) (size 1.5) (drill 1) (layers "F.Cu" "B.Cu") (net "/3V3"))
 (via (at 134.5 39.5) (size 2) (drill 1) (layers "F.Cu" "B.Cu") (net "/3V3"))
 (segment (start 148 27) (end 152.1 22.9) (width 0.9) (layer "B.Cu") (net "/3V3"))
 (segment (start 134.5 39.5) (end 134 40) (width 0.9) (layer "B.Cu") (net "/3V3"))
 (segment (start 152.1 22.9) (end 154.1 22.9) (width 0.9) (layer "B.Cu") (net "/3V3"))
 (segment (start 145 27) (end 146.5 27) (width 0.9) (layer "B.Cu") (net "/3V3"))
 (segment (start 144.5 37.5) (end 141.3 37.5) (width 0.9) (layer "B.Cu") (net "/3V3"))
 (segment (start 137.54 21.54) (end 141 25) (width 0.9) (layer "B.Cu") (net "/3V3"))
 (segment (start 146.5 27) (end 148 27) (width 0.9) (layer "B.Cu") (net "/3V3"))
 (segment (start 146.5 27) (end 146.5 35.5) (width 0.9) (layer "B.Cu") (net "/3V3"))
 (segment (start 131 46) (end 125.08 46) (width 0.9) (layer "B.Cu") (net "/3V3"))
 (segment (start 141 25) (end 143 25) (width 0.9) (layer "B.Cu") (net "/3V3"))
 (segment (start 143 25) (end 145 27) (width 0.9) (layer "B.Cu") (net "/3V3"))
 (segment (start 125.08 46) (end 123.58 47.5) (width 0.9) (layer "B.Cu") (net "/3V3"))
 (segment (start 123.58 47.5) (end 123.58 49) (width 0.9) (layer "B.Cu") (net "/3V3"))
 (segment (start 134 40) (end 134 43) (width 0.9) (layer "B.Cu") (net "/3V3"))
 (segment (start 134 43) (end 131 46) (width 0.9) (layer "B.Cu") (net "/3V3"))
 (segment (start 137.54 20.5) (end 137.54 21.54) (width 0.9) (layer "B.Cu") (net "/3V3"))
 (segment (start 146.5 35.5) (end 144.5 37.5) (width 0.9) (layer "B.Cu") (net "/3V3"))
 (segment (start 137.5 30.5) (end 136 32) (width 0.9) (layer "F.Cu") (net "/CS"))
 (segment (start 140.55 25.95) (end 137.5 29) (width 0.9) (layer "F.Cu") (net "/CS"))
 (segment (start 136 32) (end 133.74 32) (width 0.9) (layer "F.Cu") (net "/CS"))
 (segment (start 137.5 29) (end 137.5 30.5) (width 0.9) (layer "F.Cu") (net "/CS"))
 (segment (start 153.05 25.95) (end 140.55 25.95) (width 0.9) (layer "F.Cu") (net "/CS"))
 (segment (start 154.1 24.9) (end 153.05 25.95) (width 0.9) (layer "F.Cu") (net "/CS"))
 (via (at 133.74 32) (size 1.5) (drill 1) (layers "F.Cu" "B.Cu") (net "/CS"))
 (segment (start 133.12 42) (end 126.12 49) (width 0.9) (layer "F.Cu") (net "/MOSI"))
 (segment (start 144 37) (end 144 40) (width 0.9) (layer "F.Cu") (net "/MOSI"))
 (segment (start 154.1 26.9) (end 144 37) (width 0.9) (layer "F.Cu") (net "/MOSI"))
 (segment (start 142 42) (end 133.12 42) (width 0.9) (layer "F.Cu") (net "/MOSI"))
 (segment (start 144 40) (end 142 42) (width 0.9) (layer "F.Cu") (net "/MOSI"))
 (via (at 126.12 49) (size 1.5) (drill 1) (layers "F.Cu" "B.Cu") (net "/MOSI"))
 (segment (start 157 30) (end 155.9 28.9) (width 0.9) (layer "F.Cu") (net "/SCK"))
 (segment (start 144.5 45.5) (end 157 33) (width 0.9) (layer "F.Cu") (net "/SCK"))
 (segment (start 155.9 28.9) (end 154.1 28.9) (width 0.9) (layer "F.Cu") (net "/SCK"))
 (segment (start 157 33) (end 157 30) (width 0.9) (layer "F.Cu") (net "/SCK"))
 (segment (start 134.7 45.5) (end 144.5 45.5) (width 0.9) (layer "F.Cu") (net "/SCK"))
 (segment (start 131.2 49) (end 134.7 45.5) (width 0.9) (layer "F.Cu") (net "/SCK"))
 (via (at 131.2 49) (size 1.5) (drill 1) (layers "F.Cu" "B.Cu") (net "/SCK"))
 (segment (start 145.5 41.5) (end 145.5 38) (width 0.9) (layer "F.Cu") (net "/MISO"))
 (segment (start 143.5 43.5) (end 145.5 41.5) (width 0.9) (layer "F.Cu") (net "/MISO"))
 (segment (start 134.16 43.5) (end 143.5 43.5) (width 0.9) (layer "F.Cu") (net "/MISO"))
 (segment (start 128.66 49) (end 134.16 43.5) (width 0.9) (layer "F.Cu") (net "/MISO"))
 (segment (start 152.6 30.9) (end 154.1 30.9) (width 0.9) (layer "F.Cu") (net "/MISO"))
 (segment (start 145.5 38) (end 152.6 30.9) (width 0.9) (layer "F.Cu") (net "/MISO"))
 (via (at 128.66 49) (size 1.5) (drill 1) (layers "F.Cu" "B.Cu") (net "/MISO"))
 (segment (start 140.08 20.92) (end 131.2 29.8) (width 0.9) (layer "F.Cu") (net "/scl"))
 (segment (start 131.2 29.8) (end 131.2 32) (width 0.9) (layer "F.Cu") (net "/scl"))
 (segment (start 140.08 20.5) (end 140.08 20.92) (width 0.9) (layer "F.Cu") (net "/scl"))
 (via (at 131.2 32) (size 1.5) (drill 1) (layers "F.Cu" "B.Cu") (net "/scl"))
 (segment (start 142.62 18.12) (end 142.5 18) (width 0.9) (layer "F.Cu") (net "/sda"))
 (segment (start 142.62 20.5) (end 142.62 18.12) (width 0.9) (layer "F.Cu") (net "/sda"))
 (segment (start 134 18) (end 128.66 23.34) (width 0.9) (layer "F.Cu") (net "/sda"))
 (segment (start 128.66 23.34) (end 128.66 32) (width 0.9) (layer "F.Cu") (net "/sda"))
 (segment (start 142.5 18) (end 134 18) (width 0.9) (layer "F.Cu") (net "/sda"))
 (via (at 128.66 32) (size 1.5) (drill 1) (layers "F.Cu" "B.Cu") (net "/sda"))
 (segment (start 119.25 25.75) (end 119.25 23.5325) (width 0.9) (layer "F.Cu") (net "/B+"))
 (segment (start 118 27.0875) (end 118 27) (width 0.9) (layer "F.Cu") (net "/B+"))
 (segment (start 118 27) (end 119.25 25.75) (width 0.9) (layer "F.Cu") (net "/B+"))
 (segment (start 118 31.5) (end 118.5 32) (width 0.9) (layer "F.Cu") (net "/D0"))
 (segment (start 119.5875 28.9125) (end 118 30.5) (width 0.9) (layer "F.Cu") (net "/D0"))
 (segment (start 121 28.9125) (end 119.5875 28.9125) (width 0.9) (layer "F.Cu") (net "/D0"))
 (segment (start 118 30.5) (end 118 31.5) (width 0.9) (layer "F.Cu") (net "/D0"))
 (segment (start 118 28.9125) (end 118 30.5) (width 0.9) (layer "F.Cu") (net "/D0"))
 (via (at 118.5 32) (size 1.5) (drill 1) (layers "F.Cu" "B.Cu") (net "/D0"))
 (segment (start 121.75 23.5325) (end 121.75 26.3375) (width 0.9) (layer "F.Cu") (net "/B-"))
 (segment (start 121.75 26.3375) (end 121 27.0875) (width 0.9) (layer "F.Cu") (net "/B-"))
 (segment (start 139.3 37) (end 133.5 37) (width 0.9) (layer "F.Cu") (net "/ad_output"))
 (segment (start 133.5 37) (end 132.5 38) (width 0.9) (layer "F.Cu") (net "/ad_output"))
 (segment (start 121 33.5) (end 121 32) (width 0.9) (layer "F.Cu") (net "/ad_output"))
 (segment (start 141.3 35) (end 139.3 37) (width 0.9) (layer "F.Cu") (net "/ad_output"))
 (segment (start 125.5 38) (end 121 33.5) (width 0.9) (layer "F.Cu") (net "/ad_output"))
 (segment (start 132.5 38) (end 125.5 38) (width 0.9) (layer "F.Cu") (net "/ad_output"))
 (via (at 121 32) (size 1.5) (drill 1) (layers "F.Cu" "B.Cu") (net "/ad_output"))
 (segment (start 126.5 36.5) (end 123.58 33.58) (width 0.9) (layer "F.Cu") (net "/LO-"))
 (segment (start 132 36.5) (end 126.5 36.5) (width 0.9) (layer "F.Cu") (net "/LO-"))
 (segment (start 137 35.5) (end 133 35.5) (width 0.9) (layer "F.Cu") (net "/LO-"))
 (segment (start 123.58 33.58) (end 123.58 32) (width 0.9) (layer "F.Cu") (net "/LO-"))
 (segment (start 140 32.5) (end 137 35.5) (width 0.9) (layer "F.Cu") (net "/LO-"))
 (segment (start 133 35.5) (end 132 36.5) (width 0.9) (layer "F.Cu") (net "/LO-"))
 (segment (start 141.3 32.5) (end 140 32.5) (width 0.9) (layer "F.Cu") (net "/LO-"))
 (via (at 123.58 32) (size 1.5) (drill 1) (layers "F.Cu" "B.Cu") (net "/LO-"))
 (segment (start 140.5 30) (end 136.5 34) (width 0.9) (layer "F.Cu") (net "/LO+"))
 (segment (start 131.944365 35) (end 129.12 35) (width 0.9) (layer "F.Cu") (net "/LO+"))
 (segment (start 136.5 34) (end 132.944365 34) (width 0.9) (layer "F.Cu") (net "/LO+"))
 (segment (start 132.944365 34) (end 131.944365 35) (width 0.9) (layer "F.Cu") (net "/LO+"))
 (segment (start 129.12 35) (end 126.12 32) (width 0.9) (layer "F.Cu") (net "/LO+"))
 (segment (start 141.3 30) (end 140.5 30) (width 0.9) (layer "F.Cu") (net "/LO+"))
 (via (at 126.12 32) (size 1.5) (drill 1) (layers "F.Cu" "B.Cu") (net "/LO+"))
 (via (at 118.5 49) (size 1.5) (drill 1) (layers "F.Cu" "B.Cu") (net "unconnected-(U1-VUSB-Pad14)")))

